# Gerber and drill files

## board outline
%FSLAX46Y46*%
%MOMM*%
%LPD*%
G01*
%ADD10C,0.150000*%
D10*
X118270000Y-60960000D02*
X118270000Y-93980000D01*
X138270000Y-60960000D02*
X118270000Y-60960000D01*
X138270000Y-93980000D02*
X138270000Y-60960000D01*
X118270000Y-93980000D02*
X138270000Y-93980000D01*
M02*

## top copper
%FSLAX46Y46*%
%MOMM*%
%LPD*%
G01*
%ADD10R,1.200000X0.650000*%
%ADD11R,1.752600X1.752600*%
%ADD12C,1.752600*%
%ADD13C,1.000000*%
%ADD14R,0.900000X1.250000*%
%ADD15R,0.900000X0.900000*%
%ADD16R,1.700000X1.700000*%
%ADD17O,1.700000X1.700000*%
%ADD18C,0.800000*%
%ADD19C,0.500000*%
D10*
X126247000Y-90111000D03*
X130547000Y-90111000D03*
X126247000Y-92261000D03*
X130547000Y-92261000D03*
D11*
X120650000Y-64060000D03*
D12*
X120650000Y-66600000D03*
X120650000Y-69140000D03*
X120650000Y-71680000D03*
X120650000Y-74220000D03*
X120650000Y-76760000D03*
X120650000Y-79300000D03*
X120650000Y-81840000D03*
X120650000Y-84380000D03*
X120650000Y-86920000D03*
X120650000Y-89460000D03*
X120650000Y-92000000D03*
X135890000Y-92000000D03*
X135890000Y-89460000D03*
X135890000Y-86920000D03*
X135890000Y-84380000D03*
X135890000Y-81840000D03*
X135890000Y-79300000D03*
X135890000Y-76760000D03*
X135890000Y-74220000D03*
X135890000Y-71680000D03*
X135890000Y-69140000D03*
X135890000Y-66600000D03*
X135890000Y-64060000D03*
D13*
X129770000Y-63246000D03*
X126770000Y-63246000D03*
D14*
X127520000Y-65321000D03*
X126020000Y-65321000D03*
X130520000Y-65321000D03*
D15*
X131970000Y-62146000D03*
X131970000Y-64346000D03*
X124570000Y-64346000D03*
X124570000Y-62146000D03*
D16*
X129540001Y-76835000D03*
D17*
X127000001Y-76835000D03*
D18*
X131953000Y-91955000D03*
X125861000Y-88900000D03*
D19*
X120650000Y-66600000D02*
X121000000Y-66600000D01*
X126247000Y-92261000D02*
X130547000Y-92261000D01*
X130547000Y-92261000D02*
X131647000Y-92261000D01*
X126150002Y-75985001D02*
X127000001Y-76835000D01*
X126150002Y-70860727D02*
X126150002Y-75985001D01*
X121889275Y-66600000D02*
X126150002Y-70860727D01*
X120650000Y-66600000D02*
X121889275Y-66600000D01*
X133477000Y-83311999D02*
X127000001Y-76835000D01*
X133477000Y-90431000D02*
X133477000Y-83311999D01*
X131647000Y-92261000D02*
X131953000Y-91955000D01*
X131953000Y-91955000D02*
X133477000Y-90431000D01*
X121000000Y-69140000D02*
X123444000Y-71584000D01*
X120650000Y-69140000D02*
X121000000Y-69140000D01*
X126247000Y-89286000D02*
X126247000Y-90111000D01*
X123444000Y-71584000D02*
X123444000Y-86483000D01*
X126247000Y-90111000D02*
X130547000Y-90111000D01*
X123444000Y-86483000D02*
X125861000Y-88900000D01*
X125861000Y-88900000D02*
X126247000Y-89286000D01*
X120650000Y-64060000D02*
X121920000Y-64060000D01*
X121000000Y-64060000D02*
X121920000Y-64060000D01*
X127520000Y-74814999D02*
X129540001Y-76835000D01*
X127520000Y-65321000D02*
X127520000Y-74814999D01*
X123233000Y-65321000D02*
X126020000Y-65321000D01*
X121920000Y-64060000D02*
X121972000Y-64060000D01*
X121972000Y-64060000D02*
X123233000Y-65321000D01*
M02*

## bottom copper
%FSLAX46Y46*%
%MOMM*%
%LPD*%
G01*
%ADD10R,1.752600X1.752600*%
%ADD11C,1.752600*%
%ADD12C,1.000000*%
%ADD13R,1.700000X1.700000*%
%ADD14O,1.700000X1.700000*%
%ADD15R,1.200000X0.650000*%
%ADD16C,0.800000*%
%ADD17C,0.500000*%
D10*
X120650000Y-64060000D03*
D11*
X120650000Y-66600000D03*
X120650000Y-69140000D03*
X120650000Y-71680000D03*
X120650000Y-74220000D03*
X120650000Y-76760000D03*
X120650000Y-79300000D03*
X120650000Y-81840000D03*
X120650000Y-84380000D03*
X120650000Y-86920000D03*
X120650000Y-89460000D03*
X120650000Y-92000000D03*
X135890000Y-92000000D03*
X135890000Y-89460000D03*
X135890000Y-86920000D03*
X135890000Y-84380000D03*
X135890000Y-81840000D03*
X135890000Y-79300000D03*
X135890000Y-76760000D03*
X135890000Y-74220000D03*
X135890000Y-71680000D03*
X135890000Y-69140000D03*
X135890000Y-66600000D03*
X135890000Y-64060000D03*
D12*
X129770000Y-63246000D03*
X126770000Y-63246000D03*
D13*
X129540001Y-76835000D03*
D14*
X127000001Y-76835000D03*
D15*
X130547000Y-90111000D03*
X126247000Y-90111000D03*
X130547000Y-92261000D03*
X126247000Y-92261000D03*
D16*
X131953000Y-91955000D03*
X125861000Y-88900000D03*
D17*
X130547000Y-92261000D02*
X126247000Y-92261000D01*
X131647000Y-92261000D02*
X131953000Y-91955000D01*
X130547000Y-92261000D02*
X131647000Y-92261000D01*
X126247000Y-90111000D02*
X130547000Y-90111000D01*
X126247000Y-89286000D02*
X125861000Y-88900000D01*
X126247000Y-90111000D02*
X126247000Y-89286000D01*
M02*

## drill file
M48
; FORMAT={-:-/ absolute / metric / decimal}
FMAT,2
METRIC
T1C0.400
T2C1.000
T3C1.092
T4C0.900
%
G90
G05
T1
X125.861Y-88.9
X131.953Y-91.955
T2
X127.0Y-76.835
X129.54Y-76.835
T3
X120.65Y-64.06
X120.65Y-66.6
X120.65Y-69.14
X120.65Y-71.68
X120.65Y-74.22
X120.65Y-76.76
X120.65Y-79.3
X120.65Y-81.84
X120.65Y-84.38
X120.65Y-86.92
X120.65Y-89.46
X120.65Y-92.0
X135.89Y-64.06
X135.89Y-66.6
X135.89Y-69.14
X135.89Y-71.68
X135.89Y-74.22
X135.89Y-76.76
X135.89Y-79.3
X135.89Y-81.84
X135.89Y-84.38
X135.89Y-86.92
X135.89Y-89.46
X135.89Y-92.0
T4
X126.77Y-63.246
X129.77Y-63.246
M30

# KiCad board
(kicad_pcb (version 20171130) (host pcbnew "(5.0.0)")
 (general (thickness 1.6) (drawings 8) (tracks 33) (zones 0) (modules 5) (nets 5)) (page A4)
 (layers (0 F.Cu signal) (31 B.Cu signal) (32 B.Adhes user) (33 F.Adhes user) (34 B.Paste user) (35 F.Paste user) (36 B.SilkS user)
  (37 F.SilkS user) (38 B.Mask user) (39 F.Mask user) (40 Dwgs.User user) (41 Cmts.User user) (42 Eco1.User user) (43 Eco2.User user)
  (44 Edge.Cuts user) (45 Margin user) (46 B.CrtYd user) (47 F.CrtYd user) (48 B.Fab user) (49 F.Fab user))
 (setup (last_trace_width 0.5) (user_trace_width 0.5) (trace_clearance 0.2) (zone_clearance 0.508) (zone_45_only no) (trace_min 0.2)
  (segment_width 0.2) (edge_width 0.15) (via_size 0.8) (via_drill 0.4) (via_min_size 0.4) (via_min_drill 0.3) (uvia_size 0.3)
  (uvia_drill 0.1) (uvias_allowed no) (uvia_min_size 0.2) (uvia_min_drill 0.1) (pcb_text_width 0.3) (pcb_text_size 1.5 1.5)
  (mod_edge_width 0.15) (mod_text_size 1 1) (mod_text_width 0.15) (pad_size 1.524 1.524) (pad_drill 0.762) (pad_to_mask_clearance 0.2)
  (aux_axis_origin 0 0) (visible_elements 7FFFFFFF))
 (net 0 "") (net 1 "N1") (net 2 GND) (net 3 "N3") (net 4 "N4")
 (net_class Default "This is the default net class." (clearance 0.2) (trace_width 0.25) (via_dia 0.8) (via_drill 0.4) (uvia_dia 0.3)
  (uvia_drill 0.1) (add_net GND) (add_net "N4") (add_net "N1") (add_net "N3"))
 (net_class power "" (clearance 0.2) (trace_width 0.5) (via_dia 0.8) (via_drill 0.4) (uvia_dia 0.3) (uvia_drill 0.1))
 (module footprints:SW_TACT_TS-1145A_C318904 (layer F.Cu) (at 128.397 91.186)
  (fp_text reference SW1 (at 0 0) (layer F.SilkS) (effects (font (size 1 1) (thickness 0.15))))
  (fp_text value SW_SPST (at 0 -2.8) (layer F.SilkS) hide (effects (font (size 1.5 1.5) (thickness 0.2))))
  (pad 1 smd rect (at -2.15 -1.075) (size 1.2 0.65) (layers F.Cu F.Paste F.Mask) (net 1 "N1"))
  (pad 1 smd rect (at 2.15 -1.075) (size 1.2 0.65) (layers F.Cu F.Paste F.Mask) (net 1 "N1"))
  (pad 2 smd rect (at -2.15 1.075) (size 1.2 0.65) (layers F.Cu F.Paste F.Mask) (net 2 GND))
  (pad 2 smd rect (at 2.15 1.075) (size 1.2 0.65) (layers F.Cu F.Paste F.Mask) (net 2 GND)))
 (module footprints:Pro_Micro (layer F.Cu) (at 128.27 76.506)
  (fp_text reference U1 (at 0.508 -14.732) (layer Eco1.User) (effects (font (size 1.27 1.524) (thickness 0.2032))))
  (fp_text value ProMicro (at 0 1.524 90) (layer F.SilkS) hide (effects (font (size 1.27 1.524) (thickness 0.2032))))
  (pad 1 thru_hole rect (at -7.62 -12.446 270) (size 1.7526 1.7526) (drill 1.0922) (layers *.Cu *.SilkS *.Mask) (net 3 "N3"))
  (pad 2 thru_hole circle (at -7.62 -9.906 270) (size 1.7526 1.7526) (drill 1.0922) (layers *.Cu *.SilkS *.Mask) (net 2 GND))
  (pad 3 thru_hole circle (at -7.62 -7.366 270) (size 1.7526 1.7526) (drill 1.0922) (layers *.Cu *.SilkS *.Mask) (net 1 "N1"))
  (pad 4 thru_hole circle (at -7.62 -4.826 270) (size 1.7526 1.7526) (drill 1.0922) (layers *.Cu *.SilkS *.Mask))
  (pad 5 thru_hole circle (at -7.62 -2.286 270) (size 1.7526 1.7526) (drill 1.0922) (layers *.Cu *.SilkS *.Mask))
  (pad 6 thru_hole circle (at -7.62 0.254 270) (size 1.7526 1.7526) (drill 1.0922) (layers *.Cu *.SilkS *.Mask))
  (pad 7 thru_hole circle (at -7.62 2.794 270) (size 1.7526 1.7526) (drill 1.0922) (layers *.Cu *.SilkS *.Mask))
  (pad 8 thru_hole circle (at -7.62 5.334 270) (size 1.7526 1.7526) (drill 1.0922) (layers *.Cu *.SilkS *.Mask))
  (pad 9 thru_hole circle (at -7.62 7.874 270) (size 1.7526 1.7526) (drill 1.0922) (layers *.Cu *.SilkS *.Mask))
  (pad 10 thru_hole circle (at -7.62 10.414 270) (size 1.7526 1.7526) (drill 1.0922) (layers *.Cu *.SilkS *.Mask))
  (pad 11 thru_hole circle (at -7.62 12.954 270) (size 1.7526 1.7526) (drill 1.0922) (layers *.Cu *.SilkS *.Mask))
  (pad 12 thru_hole circle (at -7.62 15.494 270) (size 1.7526 1.7526) (drill 1.0922) (layers *.Cu *.SilkS *.Mask))
  (pad 24 thru_hole circle (at 7.62 15.494 270) (size 1.7526 1.7526) (drill 1.0922) (layers *.Cu *.SilkS *.Mask))
  (pad 23 thru_hole circle (at 7.62 12.954 270) (size 1.7526 1.7526) (drill 1.0922) (layers *.Cu *.SilkS *.Mask))
  (pad 22 thru_hole circle (at 7.62 10.414 270) (size 1.7526 1.7526) (drill 1.0922) (layers *.Cu *.SilkS *.Mask))
  (pad 21 thru_hole circle (at 7.62 7.874 270) (size 1.7526 1.7526) (drill 1.0922) (layers *.Cu *.SilkS *.Mask))
  (pad 20 thru_hole circle (at 7.62 5.334 270) (size 1.7526 1.7526) (drill 1.0922) (layers *.Cu *.SilkS *.Mask))
  (pad 19 thru_hole circle (at 7.62 2.794 270) (size 1.7526 1.7526) (drill 1.0922) (layers *.Cu *.SilkS *.Mask))
  (pad 18 thru_hole circle (at 7.62 0.254 270) (size 1.7526 1.7526) (drill 1.0922) (layers *.Cu *.SilkS *.Mask))
  (pad 17 thru_hole circle (at 7.62 -2.286 270) (size 1.7526 1.7526) (drill 1.0922) (layers *.Cu *.SilkS *.Mask))
  (pad 16 thru_hole circle (at 7.62 -4.826 270) (size 1.7526 1.7526) (drill 1.0922) (layers *.Cu *.SilkS *.Mask))
  (pad 15 thru_hole circle (at 7.62 -7.366 270) (size 1.7526 1.7526) (drill 1.0922) (layers *.Cu *.SilkS *.Mask))
  (pad 14 thru_hole circle (at 7.62 -9.906 270) (size 1.7526 1.7526) (drill 1.0922) (layers *.Cu *.SilkS *.Mask))
  (pad 13 thru_hole circle (at 7.62 -12.446 270) (size 1.7526 1.7526) (drill 1.0922) (layers *.Cu *.SilkS *.Mask)))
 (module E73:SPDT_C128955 (layer F.Cu) (at 128.27 63.246)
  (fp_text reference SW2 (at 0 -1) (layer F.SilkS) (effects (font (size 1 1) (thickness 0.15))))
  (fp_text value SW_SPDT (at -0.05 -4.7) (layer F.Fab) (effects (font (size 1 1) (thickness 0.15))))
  (pad "" np_thru_hole circle (at 1.5 0) (size 1 1) (drill 0.9) (layers *.Cu *.Mask))
  (pad "" np_thru_hole circle (at -1.5 0) (size 1 1) (drill 0.9) (layers *.Cu *.Mask))
  (pad 2 smd rect (at -0.75 2.075) (size 0.9 1.25) (layers F.Cu F.Paste F.Mask) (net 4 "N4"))
  (pad 3 smd rect (at -2.25 2.075) (size 0.9 1.25) (layers F.Cu F.Paste F.Mask) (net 3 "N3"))
  (pad 1 smd rect (at 2.25 2.075) (size 0.9 1.25) (layers F.Cu F.Paste F.Mask))
  (pad 0 smd rect (at 3.7 -1.1) (size 0.9 0.9) (layers F.Cu F.Paste F.Mask))
  (pad 0 smd rect (at 3.7 1.1) (size 0.9 0.9) (layers F.Cu F.Paste F.Mask))
  (pad 0 smd rect (at -3.7 1.1) (size 0.9 0.9) (layers F.Cu F.Paste F.Mask))
  (pad 0 smd rect (at -3.7 -1.1) (size 0.9 0.9) (layers F.Cu F.Paste F.Mask)))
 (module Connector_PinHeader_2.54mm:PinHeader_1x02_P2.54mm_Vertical (layer F.Cu) (at 129.540001 76.835 270)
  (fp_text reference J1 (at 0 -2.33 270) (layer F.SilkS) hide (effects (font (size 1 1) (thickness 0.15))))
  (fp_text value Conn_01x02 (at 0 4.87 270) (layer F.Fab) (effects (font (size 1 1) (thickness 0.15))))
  (pad 1 thru_hole rect (at 0 0 270) (size 1.7 1.7) (drill 1) (layers *.Cu *.Mask) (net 4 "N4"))
  (pad 2 thru_hole oval (at 0 2.54 270) (size 1.7 1.7) (drill 1) (layers *.Cu *.Mask) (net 2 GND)))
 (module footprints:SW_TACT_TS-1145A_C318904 (layer B.Cu) (at 128.397 91.186 180)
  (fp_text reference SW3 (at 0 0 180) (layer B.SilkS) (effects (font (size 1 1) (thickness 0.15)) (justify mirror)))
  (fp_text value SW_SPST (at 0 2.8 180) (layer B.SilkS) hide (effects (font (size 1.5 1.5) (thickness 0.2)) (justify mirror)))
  (pad 1 smd rect (at -2.15 1.075 180) (size 1.2 0.65) (layers B.Cu B.Paste B.Mask) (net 1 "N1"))
  (pad 1 smd rect (at 2.15 1.075 180) (size 1.2 0.65) (layers B.Cu B.Paste B.Mask) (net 1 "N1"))
  (pad 2 smd rect (at -2.15 -1.075 180) (size 1.2 0.65) (layers B.Cu B.Paste B.Mask) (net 2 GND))
  (pad 2 smd rect (at 2.15 -1.075 180) (size 1.2 0.65) (layers B.Cu B.Paste B.Mask) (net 2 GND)))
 (gr_line (start 118.27 60.96) (end 118.27 93.98) (layer Edge.Cuts) (width 0.15))
 (gr_line (start 138.27 60.96) (end 118.27 60.96) (layer Edge.Cuts) (width 0.15))
 (gr_line (start 138.27 93.98) (end 138.27 60.96) (layer Edge.Cuts) (width 0.15))
 (gr_line (start 118.27 93.98) (end 138.27 93.98) (layer Edge.Cuts) (width 0.15))
 (segment (start 120.65 66.6) (end 121 66.6) (width 0.5) (layer F.Cu) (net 2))
 (segment (start 126.247 92.261) (end 130.547 92.261) (width 0.5) (layer F.Cu) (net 2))
 (segment (start 130.547 92.261) (end 131.647 92.261) (width 0.5) (layer F.Cu) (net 2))
 (segment (start 126.150002 75.985001) (end 127.000001 76.835) (width 0.5) (layer F.Cu) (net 2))
 (segment (start 126.150002 70.860727) (end 126.150002 75.985001) (width 0.5) (layer F.Cu) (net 2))
 (segment (start 121.889275 66.6) (end 126.150002 70.860727) (width 0.5) (layer F.Cu) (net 2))
 (segment (start 120.65 66.6) (end 121.889275 66.6) (width 0.5) (layer F.Cu) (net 2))
 (segment (start 133.477 83.311999) (end 127.000001 76.835) (width 0.5) (layer F.Cu) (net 2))
 (segment (start 133.477 90.431) (end 133.477 83.311999) (width 0.5) (layer F.Cu) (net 2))
 (segment (start 130.547 92.261) (end 126.247 92.261) (width 0.5) (layer B.Cu) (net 2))
 (via (at 131.953 91.955) (size 0.8) (drill 0.4) (layers F.Cu B.Cu) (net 2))
 (segment (start 131.647 92.261) (end 131.953 91.955) (width 0.5) (layer B.Cu) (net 2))
 (segment (start 130.547 92.261) (end 131.647 92.261) (width 0.5) (layer B.Cu) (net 2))
 (segment (start 131.647 92.261) (end 131.953 91.955) (width 0.5) (layer F.Cu) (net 2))
 (segment (start 131.953 91.955) (end 133.477 90.431) (width 0.5) (layer F.Cu) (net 2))
 (segment (start 121 69.14) (end 123.444 71.584) (width 0.5) (layer F.Cu) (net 1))
 (segment (start 120.65 69.14) (end 121 69.14) (width 0.5) (layer F.Cu) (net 1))
 (segment (start 126.247 89.286) (end 126.247 90.111) (width 0.5) (layer F.Cu) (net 1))
 (segment (start 123.444 71.584) (end 123.444 86.483) (width 0.5) (layer F.Cu) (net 1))
 (segment (start 126.247 90.111) (end 130.547 90.111) (width 0.5) (layer F.Cu) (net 1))
 (segment (start 126.247 90.111) (end 130.547 90.111) (width 0.5) (layer B.Cu) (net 1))
 (via (at 125.861 88.9) (size 0.8) (drill 0.4) (layers F.Cu B.Cu) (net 1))
 (segment (start 126.247 89.286) (end 125.861 88.9) (width 0.5) (layer B.Cu) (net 1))
 (segment (start 126.247 90.111) (end 126.247 89.286) (width 0.5) (layer B.Cu) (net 1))
 (segment (start 123.444 86.483) (end 125.861 88.9) (width 0.5) (layer F.Cu) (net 1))
 (segment (start 125.861 88.9) (end 126.247 89.286) (width 0.5) (layer F.Cu) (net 1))
 (segment (start 120.65 64.06) (end 121.92 64.06) (width 0.5) (layer F.Cu) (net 3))
 (segment (start 121 64.06) (end 121.92 64.06) (width 0.5) (layer F.Cu) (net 3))
 (segment (start 127.52 74.814999) (end 129.540001 76.835) (width 0.5) (layer F.Cu) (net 4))
 (segment (start 127.52 65.321) (end 127.52 74.814999) (width 0.5) (layer F.Cu) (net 4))
 (segment (start 123.233 65.321) (end 126.02 65.321) (width 0.5) (layer F.Cu) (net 3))
 (segment (start 121.92 64.06) (end 121.972 64.06) (width 0.5) (layer F.Cu) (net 3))
 (segment (start 121.972 64.06) (end 123.233 65.321) (width 0.5) (layer F.Cu) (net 3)))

